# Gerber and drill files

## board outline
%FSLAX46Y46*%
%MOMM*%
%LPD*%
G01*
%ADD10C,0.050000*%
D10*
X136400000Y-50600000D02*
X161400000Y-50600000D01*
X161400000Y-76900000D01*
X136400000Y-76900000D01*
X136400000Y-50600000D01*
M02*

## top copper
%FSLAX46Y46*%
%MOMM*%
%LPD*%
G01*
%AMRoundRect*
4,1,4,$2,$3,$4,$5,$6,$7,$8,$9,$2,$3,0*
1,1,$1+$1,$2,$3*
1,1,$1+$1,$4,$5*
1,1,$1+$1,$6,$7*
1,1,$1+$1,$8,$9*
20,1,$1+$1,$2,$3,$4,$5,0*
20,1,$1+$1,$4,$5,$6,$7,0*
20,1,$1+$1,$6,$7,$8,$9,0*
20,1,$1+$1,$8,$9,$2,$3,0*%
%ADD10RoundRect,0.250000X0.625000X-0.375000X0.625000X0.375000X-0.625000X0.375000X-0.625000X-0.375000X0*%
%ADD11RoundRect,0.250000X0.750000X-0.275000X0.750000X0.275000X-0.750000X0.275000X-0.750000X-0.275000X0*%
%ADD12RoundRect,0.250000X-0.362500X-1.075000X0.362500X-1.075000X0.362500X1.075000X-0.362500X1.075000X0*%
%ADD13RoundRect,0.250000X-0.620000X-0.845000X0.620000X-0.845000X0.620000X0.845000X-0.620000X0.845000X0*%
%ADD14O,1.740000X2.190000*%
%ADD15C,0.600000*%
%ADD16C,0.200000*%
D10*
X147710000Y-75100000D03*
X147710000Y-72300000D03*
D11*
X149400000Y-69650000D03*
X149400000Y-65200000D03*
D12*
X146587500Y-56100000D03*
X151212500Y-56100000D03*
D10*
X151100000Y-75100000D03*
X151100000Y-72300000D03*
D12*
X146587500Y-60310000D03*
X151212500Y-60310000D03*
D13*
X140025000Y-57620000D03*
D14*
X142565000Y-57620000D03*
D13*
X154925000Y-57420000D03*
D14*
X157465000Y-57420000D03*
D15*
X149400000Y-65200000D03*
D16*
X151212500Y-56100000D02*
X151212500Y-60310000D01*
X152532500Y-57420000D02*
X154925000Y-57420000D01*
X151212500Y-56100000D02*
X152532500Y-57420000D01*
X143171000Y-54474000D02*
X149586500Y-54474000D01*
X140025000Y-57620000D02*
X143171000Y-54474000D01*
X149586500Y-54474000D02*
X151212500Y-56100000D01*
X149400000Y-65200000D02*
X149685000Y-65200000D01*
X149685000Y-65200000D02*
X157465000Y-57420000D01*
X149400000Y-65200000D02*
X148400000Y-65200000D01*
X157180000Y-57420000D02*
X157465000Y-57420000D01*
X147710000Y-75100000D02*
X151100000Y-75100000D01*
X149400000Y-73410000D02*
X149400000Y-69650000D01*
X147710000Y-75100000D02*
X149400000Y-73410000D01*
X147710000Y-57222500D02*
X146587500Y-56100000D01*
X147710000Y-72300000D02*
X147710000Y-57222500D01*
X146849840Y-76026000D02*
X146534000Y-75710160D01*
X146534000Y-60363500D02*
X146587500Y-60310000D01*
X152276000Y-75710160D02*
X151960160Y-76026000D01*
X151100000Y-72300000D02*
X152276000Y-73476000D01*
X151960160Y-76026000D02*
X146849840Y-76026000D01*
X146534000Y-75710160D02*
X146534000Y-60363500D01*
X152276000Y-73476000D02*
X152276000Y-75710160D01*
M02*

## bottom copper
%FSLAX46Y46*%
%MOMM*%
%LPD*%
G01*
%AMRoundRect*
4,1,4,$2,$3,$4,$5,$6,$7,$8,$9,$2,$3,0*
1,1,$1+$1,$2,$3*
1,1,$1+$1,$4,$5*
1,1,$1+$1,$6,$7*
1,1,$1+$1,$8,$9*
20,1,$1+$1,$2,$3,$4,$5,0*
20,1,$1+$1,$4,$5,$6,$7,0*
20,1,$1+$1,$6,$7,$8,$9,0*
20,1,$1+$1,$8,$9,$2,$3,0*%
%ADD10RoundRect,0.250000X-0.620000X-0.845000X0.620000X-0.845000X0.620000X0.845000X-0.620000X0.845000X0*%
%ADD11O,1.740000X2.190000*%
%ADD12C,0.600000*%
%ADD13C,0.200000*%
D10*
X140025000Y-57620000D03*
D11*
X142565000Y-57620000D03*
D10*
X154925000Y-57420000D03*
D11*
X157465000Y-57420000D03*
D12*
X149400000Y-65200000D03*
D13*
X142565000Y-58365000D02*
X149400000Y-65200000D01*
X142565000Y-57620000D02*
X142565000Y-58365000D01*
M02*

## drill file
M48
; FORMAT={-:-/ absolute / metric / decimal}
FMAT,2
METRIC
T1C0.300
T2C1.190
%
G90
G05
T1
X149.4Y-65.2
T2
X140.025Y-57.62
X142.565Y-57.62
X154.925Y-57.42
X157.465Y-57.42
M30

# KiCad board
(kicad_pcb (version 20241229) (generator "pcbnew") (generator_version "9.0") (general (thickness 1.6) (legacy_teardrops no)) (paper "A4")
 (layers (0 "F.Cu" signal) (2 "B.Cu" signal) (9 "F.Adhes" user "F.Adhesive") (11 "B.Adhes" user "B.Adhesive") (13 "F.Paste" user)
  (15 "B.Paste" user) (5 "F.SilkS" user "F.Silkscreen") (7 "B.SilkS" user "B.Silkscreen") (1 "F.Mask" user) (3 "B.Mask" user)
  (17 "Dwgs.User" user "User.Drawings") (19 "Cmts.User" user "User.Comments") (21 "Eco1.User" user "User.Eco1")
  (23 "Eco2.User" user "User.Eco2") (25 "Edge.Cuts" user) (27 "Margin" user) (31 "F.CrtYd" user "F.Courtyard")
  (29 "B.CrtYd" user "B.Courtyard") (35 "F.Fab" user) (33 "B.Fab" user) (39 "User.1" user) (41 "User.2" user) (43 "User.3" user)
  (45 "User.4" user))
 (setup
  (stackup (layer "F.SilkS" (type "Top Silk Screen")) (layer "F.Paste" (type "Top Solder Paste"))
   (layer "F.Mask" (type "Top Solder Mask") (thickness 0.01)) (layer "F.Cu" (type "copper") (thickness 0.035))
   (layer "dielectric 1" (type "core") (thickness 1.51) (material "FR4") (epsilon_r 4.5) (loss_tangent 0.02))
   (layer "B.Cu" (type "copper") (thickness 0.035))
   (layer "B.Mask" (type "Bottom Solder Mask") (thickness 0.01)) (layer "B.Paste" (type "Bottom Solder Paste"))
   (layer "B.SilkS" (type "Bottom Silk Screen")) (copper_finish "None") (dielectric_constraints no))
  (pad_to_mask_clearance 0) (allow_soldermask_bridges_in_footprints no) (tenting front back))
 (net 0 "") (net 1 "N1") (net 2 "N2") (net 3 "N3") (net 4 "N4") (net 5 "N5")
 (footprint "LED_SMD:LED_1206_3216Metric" (layer "F.Cu") (at 147.71 73.7 90)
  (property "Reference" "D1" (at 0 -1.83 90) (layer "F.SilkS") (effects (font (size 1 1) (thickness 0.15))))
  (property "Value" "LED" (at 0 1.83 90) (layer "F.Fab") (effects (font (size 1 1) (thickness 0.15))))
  (pad "1" smd roundrect (at -1.4 0 90) (size 1.25 1.75) (layers "F.Cu" "F.Mask" "F.Paste") (roundrect_rratio 0.2) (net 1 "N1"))
  (pad "2" smd roundrect (at 1.4 0 90) (size 1.25 1.75) (layers "F.Cu" "F.Mask" "F.Paste") (roundrect_rratio 0.2) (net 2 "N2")))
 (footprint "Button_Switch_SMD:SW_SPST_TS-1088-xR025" (layer "F.Cu") (at 149.4 67.425 90)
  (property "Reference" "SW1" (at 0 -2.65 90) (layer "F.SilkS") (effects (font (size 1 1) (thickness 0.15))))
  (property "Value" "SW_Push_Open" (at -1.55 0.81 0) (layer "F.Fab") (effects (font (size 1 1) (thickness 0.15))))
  (pad "1" smd roundrect (at -2.225 0 90) (size 1.05 2) (layers "F.Cu" "F.Mask" "F.Paste") (roundrect_rratio 0.2380952381) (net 1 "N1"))
  (pad "2" smd roundrect (at 2.225 0 90) (size 1.05 2) (layers "F.Cu" "F.Mask" "F.Paste") (roundrect_rratio 0.2380952381) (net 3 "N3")))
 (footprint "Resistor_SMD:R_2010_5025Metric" (layer "F.Cu") (at 148.9 56.1)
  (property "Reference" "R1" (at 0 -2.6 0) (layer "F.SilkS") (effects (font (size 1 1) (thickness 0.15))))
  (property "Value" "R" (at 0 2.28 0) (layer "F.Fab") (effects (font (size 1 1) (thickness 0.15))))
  (pad "1" smd roundrect (at -2.3125 0) (size 1.225 2.65) (layers "F.Cu" "F.Mask" "F.Paste") (roundrect_rratio 0.204082) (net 2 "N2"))
  (pad "2" smd roundrect (at 2.3125 0) (size 1.225 2.65) (layers "F.Cu" "F.Mask" "F.Paste") (roundrect_rratio 0.204082) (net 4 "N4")))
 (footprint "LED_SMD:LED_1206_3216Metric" (layer "F.Cu") (at 151.1 73.7 90)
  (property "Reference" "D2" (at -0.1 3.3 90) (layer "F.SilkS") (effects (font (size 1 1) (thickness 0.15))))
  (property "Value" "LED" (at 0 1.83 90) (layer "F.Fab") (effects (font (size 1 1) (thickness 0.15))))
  (pad "1" smd roundrect (at -1.4 0 90) (size 1.25 1.75) (layers "F.Cu" "F.Mask" "F.Paste") (roundrect_rratio 0.2) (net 1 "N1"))
  (pad "2" smd roundrect (at 1.4 0 90) (size 1.25 1.75) (layers "F.Cu" "F.Mask" "F.Paste") (roundrect_rratio 0.2) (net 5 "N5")))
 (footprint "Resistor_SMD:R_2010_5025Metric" (layer "F.Cu") (at 148.9 60.31)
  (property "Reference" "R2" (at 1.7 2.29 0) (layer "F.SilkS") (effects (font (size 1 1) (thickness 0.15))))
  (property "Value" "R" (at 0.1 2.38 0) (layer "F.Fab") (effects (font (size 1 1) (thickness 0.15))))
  (pad "1" smd roundrect (at -2.3125 0) (size 1.225 2.65) (layers "F.Cu" "F.Mask" "F.Paste") (roundrect_rratio 0.204082) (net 5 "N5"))
  (pad "2" smd roundrect (at 2.3125 0) (size 1.225 2.65) (layers "F.Cu" "F.Mask" "F.Paste") (roundrect_rratio 0.204082) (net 4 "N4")))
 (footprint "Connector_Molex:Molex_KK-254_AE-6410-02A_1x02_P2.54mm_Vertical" (layer "F.Cu") (at 140.025 57.62)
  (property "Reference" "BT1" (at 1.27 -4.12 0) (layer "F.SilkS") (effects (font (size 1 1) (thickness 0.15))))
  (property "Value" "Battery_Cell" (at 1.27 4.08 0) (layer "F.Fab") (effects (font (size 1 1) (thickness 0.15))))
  (pad "1" thru_hole roundrect (at 0 0) (size 1.74 2.19) (drill 1.19) (layers "*.Cu" "*.Mask") (remove_unused_layers no)
   (roundrect_rratio 0.143678) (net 4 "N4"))
  (pad "2" thru_hole oval (at 2.54 0) (size 1.74 2.19) (drill 1.19) (layers "*.Cu" "*.Mask") (remove_unused_layers no) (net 3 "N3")))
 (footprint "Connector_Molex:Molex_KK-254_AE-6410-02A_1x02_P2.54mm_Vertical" (layer "F.Cu") (at 154.925 57.42)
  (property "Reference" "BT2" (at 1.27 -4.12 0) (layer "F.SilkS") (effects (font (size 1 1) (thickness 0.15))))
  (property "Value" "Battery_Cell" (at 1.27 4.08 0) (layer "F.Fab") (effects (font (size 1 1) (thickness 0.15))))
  (pad "1" thru_hole roundrect (at 0 0) (size 1.74 2.19) (drill 1.19) (layers "*.Cu" "*.Mask") (remove_unused_layers no)
   (roundrect_rratio 0.143678) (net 4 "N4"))
  (pad "2" thru_hole oval (at 2.54 0) (size 1.74 2.19) (drill 1.19) (layers "*.Cu" "*.Mask") (remove_unused_layers no) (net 3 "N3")))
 (gr_rect (start 136.4 50.6) (end 161.4 76.9) (stroke (width 0.05) (type default)) (fill no) (layer "Edge.Cuts"))
 (segment (start 151.2125 56.1) (end 151.2125 60.31) (width 0.2) (layer "F.Cu") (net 4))
 (segment (start 152.5325 57.42) (end 154.925 57.42) (width 0.2) (layer "F.Cu") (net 4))
 (segment (start 151.2125 56.1) (end 152.5325 57.42) (width 0.2) (layer "F.Cu") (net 4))
 (segment (start 143.171 54.474) (end 149.5865 54.474) (width 0.2) (layer "F.Cu") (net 4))
 (segment (start 140.025 57.62) (end 143.171 54.474) (width 0.2) (layer "F.Cu") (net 4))
 (segment (start 149.5865 54.474) (end 151.2125 56.1) (width 0.2) (layer "F.Cu") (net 4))
 (segment (start 149.4 65.2) (end 149.685 65.2) (width 0.2) (layer "F.Cu") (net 3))
 (segment (start 149.685 65.2) (end 157.465 57.42) (width 0.2) (layer "F.Cu") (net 3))
 (segment (start 149.4 65.2) (end 148.4 65.2) (width 0.2) (layer "F.Cu") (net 3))
 (segment (start 157.18 57.42) (end 157.465 57.42) (width 0.2) (layer "F.Cu") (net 3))
 (via (at 149.4 65.2) (size 0.6) (drill 0.3) (layers "F.Cu" "B.Cu") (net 3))
 (segment (start 142.565 58.365) (end 149.4 65.2) (width 0.2) (layer "B.Cu") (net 3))
 (segment (start 142.565 57.62) (end 142.565 58.365) (width 0.2) (layer "B.Cu") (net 3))
 (segment (start 147.71 75.1) (end 151.1 75.1) (width 0.2) (layer "F.Cu") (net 1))
 (segment (start 149.4 73.41) (end 149.4 69.65) (width 0.2) (layer "F.Cu") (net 1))
 (segment (start 147.71 75.1) (end 149.4 73.41) (width 0.2) (layer "F.Cu") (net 1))
 (segment (start 147.71 57.2225) (end 146.5875 56.1) (width 0.2) (layer "F.Cu") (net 2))
 (segment (start 147.71 72.3) (end 147.71 57.2225) (width 0.2) (layer "F.Cu") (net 2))
 (segment (start 146.84984 76.026) (end 146.534 75.71016) (width 0.2) (layer "F.Cu") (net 5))
 (segment (start 146.534 60.3635) (end 146.5875 60.31) (width 0.2) (layer "F.Cu") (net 5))
 (segment (start 152.276 75.71016) (end 151.96016 76.026) (width 0.2) (layer "F.Cu") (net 5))
 (segment (start 151.1 72.3) (end 152.276 73.476) (width 0.2) (layer "F.Cu") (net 5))
 (segment (start 151.96016 76.026) (end 146.84984 76.026) (width 0.2) (layer "F.Cu") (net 5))
 (segment (start 146.534 75.71016) (end 146.534 60.3635) (width 0.2) (layer "F.Cu") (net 5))
 (segment (start 152.276 73.476) (end 152.276 75.71016) (width 0.2) (layer "F.Cu") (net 5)))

